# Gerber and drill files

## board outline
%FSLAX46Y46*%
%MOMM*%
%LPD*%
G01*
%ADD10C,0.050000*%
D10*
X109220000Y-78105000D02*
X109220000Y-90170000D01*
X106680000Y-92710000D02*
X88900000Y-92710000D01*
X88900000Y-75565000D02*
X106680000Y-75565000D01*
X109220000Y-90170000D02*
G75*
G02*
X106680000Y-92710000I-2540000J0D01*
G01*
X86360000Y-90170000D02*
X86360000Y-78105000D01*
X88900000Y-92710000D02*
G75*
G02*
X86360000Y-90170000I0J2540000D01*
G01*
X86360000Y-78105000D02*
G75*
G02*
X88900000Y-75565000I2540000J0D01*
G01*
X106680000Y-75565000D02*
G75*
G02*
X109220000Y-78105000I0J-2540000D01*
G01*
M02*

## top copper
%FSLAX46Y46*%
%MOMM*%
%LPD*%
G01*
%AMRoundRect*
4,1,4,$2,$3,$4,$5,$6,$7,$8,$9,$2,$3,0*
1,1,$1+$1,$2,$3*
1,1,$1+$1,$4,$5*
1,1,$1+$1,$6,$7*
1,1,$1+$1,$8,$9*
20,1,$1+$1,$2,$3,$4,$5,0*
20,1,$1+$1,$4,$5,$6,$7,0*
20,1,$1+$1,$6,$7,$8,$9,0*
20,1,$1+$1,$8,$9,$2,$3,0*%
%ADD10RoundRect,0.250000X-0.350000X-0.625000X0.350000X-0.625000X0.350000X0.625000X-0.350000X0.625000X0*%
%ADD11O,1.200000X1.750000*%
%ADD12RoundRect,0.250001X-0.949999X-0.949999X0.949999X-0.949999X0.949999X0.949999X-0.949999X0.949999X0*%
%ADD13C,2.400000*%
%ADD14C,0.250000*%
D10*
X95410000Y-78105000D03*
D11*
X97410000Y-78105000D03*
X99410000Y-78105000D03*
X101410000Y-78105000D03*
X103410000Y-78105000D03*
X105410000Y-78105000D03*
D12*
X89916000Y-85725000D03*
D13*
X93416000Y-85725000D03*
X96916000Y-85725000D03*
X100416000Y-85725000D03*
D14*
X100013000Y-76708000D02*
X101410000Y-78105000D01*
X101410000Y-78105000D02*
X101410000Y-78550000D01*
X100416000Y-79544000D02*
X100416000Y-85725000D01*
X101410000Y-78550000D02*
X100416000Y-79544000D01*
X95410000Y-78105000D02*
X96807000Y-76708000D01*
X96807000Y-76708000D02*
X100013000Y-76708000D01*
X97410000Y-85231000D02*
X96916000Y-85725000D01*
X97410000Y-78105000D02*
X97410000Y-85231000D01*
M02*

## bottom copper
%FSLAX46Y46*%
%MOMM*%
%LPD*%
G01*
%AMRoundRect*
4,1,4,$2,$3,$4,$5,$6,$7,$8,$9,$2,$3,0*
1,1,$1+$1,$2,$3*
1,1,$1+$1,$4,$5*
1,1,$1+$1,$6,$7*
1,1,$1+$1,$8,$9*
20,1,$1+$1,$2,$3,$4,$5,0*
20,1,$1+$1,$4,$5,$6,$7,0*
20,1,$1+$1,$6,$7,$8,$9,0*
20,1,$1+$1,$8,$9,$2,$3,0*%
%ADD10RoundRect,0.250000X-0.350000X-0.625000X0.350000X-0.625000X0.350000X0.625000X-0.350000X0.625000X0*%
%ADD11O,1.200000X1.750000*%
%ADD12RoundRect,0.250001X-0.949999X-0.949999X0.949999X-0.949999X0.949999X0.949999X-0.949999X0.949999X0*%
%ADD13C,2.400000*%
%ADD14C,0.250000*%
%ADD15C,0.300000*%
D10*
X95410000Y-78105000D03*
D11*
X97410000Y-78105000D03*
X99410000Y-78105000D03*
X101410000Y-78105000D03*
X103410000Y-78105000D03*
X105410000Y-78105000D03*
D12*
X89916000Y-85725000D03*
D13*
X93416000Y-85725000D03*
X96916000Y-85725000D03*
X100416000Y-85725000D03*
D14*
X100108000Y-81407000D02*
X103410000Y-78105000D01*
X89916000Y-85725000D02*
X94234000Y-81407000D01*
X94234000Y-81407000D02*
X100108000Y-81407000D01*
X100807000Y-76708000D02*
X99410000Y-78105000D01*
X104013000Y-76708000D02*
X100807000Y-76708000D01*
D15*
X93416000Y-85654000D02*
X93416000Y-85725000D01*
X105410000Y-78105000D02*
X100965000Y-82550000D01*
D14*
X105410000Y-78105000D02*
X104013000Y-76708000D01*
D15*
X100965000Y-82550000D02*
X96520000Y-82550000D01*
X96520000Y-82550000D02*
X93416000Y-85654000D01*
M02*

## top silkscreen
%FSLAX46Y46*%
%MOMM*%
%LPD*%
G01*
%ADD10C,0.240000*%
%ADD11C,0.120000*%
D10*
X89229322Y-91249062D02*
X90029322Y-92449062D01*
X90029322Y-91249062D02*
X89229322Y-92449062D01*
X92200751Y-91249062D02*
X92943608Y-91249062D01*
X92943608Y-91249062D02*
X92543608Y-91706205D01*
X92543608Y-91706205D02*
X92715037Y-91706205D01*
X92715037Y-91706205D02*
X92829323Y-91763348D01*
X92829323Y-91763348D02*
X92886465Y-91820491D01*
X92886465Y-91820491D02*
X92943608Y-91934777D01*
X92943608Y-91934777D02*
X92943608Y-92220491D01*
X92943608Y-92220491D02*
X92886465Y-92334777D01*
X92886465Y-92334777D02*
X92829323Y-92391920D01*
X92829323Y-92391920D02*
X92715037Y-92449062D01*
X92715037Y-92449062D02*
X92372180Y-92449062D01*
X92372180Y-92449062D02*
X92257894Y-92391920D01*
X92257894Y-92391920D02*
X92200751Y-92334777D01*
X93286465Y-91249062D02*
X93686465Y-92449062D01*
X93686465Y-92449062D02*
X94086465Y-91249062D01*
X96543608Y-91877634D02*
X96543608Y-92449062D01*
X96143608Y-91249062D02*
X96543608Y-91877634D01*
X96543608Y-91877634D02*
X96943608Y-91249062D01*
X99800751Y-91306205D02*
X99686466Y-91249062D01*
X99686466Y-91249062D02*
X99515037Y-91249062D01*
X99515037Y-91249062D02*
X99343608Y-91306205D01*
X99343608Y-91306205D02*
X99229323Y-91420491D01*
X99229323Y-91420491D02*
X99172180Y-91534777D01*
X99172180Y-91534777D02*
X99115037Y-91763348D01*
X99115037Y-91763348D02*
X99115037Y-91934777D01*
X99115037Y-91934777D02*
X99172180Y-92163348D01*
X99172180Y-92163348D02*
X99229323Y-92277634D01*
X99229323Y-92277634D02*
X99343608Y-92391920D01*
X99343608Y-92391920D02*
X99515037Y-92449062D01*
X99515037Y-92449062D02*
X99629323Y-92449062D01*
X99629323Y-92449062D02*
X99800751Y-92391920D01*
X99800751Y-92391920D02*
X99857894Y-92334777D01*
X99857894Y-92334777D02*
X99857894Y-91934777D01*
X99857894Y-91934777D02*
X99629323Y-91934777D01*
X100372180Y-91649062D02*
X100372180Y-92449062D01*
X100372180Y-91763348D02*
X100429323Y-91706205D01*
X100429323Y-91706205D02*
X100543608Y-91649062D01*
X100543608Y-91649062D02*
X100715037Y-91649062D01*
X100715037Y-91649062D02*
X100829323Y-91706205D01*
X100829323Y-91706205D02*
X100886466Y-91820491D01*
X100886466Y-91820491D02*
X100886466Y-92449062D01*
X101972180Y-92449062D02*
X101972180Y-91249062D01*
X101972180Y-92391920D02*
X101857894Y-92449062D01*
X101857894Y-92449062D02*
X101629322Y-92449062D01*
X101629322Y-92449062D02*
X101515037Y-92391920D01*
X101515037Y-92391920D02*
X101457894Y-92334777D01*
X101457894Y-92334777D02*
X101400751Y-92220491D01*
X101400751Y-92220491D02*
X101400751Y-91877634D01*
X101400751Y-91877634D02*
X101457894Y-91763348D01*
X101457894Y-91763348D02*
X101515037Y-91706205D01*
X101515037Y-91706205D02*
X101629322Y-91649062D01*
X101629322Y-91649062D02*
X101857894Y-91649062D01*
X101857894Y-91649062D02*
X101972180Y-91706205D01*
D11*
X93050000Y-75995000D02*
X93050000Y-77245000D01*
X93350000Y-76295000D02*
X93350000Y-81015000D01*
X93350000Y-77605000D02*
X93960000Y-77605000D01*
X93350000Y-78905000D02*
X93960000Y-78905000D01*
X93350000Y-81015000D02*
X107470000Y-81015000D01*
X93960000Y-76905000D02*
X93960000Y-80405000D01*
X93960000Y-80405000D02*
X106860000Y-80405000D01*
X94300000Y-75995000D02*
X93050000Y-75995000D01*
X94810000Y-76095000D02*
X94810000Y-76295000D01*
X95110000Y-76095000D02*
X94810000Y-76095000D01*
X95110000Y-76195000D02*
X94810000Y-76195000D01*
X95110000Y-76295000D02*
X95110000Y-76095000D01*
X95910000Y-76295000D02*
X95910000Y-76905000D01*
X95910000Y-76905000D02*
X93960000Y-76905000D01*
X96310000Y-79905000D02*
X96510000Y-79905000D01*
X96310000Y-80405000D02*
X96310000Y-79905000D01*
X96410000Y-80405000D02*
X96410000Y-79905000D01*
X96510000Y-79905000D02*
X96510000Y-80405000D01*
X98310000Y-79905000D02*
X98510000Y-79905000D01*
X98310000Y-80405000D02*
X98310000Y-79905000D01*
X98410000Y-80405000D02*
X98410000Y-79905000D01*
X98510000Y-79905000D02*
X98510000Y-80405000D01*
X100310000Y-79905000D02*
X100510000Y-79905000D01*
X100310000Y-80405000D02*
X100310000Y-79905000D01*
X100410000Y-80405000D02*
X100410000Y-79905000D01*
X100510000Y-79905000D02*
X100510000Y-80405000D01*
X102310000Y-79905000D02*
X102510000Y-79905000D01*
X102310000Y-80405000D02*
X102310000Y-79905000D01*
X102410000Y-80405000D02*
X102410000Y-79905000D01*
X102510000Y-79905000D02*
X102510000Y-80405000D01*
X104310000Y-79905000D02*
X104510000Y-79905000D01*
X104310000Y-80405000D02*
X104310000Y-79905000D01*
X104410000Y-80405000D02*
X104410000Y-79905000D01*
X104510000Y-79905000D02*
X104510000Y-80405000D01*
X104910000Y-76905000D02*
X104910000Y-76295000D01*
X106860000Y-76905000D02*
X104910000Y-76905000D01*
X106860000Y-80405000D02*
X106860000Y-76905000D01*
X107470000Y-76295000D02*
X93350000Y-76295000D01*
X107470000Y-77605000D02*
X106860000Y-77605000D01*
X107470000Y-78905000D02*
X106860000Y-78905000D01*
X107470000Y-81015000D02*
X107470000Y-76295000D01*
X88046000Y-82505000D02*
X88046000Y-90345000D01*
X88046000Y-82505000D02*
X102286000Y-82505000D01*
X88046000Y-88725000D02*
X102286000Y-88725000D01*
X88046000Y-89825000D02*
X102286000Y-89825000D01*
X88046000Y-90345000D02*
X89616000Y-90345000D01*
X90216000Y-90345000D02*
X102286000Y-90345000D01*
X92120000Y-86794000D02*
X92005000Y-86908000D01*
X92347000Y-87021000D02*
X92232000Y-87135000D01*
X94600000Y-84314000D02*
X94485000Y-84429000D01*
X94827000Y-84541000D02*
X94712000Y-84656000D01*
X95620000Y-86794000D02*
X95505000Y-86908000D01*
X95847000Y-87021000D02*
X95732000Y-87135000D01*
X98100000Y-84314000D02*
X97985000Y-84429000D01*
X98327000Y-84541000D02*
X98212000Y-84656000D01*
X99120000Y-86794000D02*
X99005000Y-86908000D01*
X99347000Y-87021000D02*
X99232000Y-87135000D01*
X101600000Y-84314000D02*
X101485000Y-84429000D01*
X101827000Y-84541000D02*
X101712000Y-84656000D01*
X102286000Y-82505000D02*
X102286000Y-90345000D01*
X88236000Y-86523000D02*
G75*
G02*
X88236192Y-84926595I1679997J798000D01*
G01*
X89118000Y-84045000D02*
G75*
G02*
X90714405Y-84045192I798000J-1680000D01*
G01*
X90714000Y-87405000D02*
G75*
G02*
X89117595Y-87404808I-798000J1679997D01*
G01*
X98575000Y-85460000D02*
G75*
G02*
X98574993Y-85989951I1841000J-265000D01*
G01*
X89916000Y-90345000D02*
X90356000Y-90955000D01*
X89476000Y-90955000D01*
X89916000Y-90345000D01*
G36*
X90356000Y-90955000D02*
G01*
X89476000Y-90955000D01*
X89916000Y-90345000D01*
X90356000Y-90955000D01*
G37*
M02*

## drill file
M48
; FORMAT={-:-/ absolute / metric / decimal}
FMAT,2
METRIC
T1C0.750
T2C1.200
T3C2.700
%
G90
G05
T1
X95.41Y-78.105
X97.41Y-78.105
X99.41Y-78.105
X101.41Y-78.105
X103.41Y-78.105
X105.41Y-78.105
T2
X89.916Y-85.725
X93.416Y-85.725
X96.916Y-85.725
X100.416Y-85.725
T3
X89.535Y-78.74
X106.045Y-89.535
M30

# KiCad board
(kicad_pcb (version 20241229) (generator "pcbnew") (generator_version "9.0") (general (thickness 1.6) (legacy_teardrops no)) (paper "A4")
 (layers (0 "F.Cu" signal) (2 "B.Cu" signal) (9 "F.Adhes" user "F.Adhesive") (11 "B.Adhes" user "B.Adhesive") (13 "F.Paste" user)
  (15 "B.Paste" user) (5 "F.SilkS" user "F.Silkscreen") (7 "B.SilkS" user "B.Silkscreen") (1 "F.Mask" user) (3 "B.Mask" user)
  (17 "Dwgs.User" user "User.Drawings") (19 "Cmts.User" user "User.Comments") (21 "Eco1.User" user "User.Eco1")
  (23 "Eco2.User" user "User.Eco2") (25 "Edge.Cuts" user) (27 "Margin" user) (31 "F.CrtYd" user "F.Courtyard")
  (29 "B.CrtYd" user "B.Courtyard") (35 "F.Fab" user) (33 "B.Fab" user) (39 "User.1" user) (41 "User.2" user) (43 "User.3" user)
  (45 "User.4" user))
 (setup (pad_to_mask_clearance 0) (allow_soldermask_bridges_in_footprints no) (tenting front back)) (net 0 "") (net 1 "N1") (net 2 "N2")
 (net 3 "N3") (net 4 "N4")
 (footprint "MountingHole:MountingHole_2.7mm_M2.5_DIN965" (layer "F.Cu") (at 89.535 78.74)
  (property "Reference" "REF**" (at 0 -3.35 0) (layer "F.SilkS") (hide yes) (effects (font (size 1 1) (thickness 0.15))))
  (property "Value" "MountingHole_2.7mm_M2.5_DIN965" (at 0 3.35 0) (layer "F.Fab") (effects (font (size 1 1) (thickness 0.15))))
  (pad "" np_thru_hole circle (at 0 0) (size 2.7 2.7) (drill 2.7) (layers "*.Cu" "*.Mask")))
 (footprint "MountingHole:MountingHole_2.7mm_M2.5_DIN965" (layer "F.Cu") (at 106.045 89.535)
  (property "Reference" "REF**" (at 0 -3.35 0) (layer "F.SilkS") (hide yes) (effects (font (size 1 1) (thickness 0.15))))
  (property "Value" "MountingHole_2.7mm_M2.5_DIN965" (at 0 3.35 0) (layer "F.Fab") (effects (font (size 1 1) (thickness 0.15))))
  (pad "" np_thru_hole circle (at 0 0) (size 2.7 2.7) (drill 2.7) (layers "*.Cu" "*.Mask")))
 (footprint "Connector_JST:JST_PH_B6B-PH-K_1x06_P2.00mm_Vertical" (layer "F.Cu") (at 95.41 78.105)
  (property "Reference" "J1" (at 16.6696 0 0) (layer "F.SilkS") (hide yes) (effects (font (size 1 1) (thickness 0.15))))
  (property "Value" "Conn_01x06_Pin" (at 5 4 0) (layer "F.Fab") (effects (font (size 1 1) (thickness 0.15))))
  (fp_line (start -2.36 -2.11) (end -2.36 -0.86) (stroke (width 0.12) (type solid)) (layer "F.SilkS"))
  (fp_line (start -2.06 -1.81) (end -2.06 2.91) (stroke (width 0.12) (type solid)) (layer "F.SilkS"))
  (fp_line (start -2.06 -0.5) (end -1.45 -0.5) (stroke (width 0.12) (type solid)) (layer "F.SilkS"))
  (fp_line (start -2.06 0.8) (end -1.45 0.8) (stroke (width 0.12) (type solid)) (layer "F.SilkS"))
  (fp_line (start -2.06 2.91) (end 12.06 2.91) (stroke (width 0.12) (type solid)) (layer "F.SilkS"))
  (fp_line (start -1.45 -1.2) (end -1.45 2.3) (stroke (width 0.12) (type solid)) (layer "F.SilkS"))
  (fp_line (start -1.45 2.3) (end 11.45 2.3) (stroke (width 0.12) (type solid)) (layer "F.SilkS"))
  (fp_line (start -1.11 -2.11) (end -2.36 -2.11) (stroke (width 0.12) (type solid)) (layer "F.SilkS"))
  (fp_line (start -0.6 -2.01) (end -0.6 -1.81) (stroke (width 0.12) (type solid)) (layer "F.SilkS"))
  (fp_line (start -0.3 -2.01) (end -0.6 -2.01) (stroke (width 0.12) (type solid)) (layer "F.SilkS"))
  (fp_line (start -0.3 -1.91) (end -0.6 -1.91) (stroke (width 0.12) (type solid)) (layer "F.SilkS"))
  (fp_line (start -0.3 -1.81) (end -0.3 -2.01) (stroke (width 0.12) (type solid)) (layer "F.SilkS"))
  (fp_line (start 0.5 -1.81) (end 0.5 -1.2) (stroke (width 0.12) (type solid)) (layer "F.SilkS"))
  (fp_line (start 0.5 -1.2) (end -1.45 -1.2) (stroke (width 0.12) (type solid)) (layer "F.SilkS"))
  (fp_line (start 0.9 1.8) (end 1.1 1.8) (stroke (width 0.12) (type solid)) (layer "F.SilkS"))
  (fp_line (start 0.9 2.3) (end 0.9 1.8) (stroke (width 0.12) (type solid)) (layer "F.SilkS"))
  (fp_line (start 1 2.3) (end 1 1.8) (stroke (width 0.12) (type solid)) (layer "F.SilkS"))
  (fp_line (start 1.1 1.8) (end 1.1 2.3) (stroke (width 0.12) (type solid)) (layer "F.SilkS"))
  (fp_line (start 2.9 1.8) (end 3.1 1.8) (stroke (width 0.12) (type solid)) (layer "F.SilkS"))
  (fp_line (start 2.9 2.3) (end 2.9 1.8) (stroke (width 0.12) (type solid)) (layer "F.SilkS"))
  (fp_line (start 3 2.3) (end 3 1.8) (stroke (width 0.12) (type solid)) (layer "F.SilkS"))
  (fp_line (start 3.1 1.8) (end 3.1 2.3) (stroke (width 0.12) (type solid)) (layer "F.SilkS"))
  (fp_line (start 4.9 1.8) (end 5.1 1.8) (stroke (width 0.12) (type solid)) (layer "F.SilkS"))
  (fp_line (start 4.9 2.3) (end 4.9 1.8) (stroke (width 0.12) (type solid)) (layer "F.SilkS"))
  (fp_line (start 5 2.3) (end 5 1.8) (stroke (width 0.12) (type solid)) (layer "F.SilkS"))
  (fp_line (start 5.1 1.8) (end 5.1 2.3) (stroke (width 0.12) (type solid)) (layer "F.SilkS"))
  (fp_line (start 6.9 1.8) (end 7.1 1.8) (stroke (width 0.12) (type solid)) (layer "F.SilkS"))
  (fp_line (start 6.9 2.3) (end 6.9 1.8) (stroke (width 0.12) (type solid)) (layer "F.SilkS"))
  (fp_line (start 7 2.3) (end 7 1.8) (stroke (width 0.12) (type solid)) (layer "F.SilkS"))
  (fp_line (start 7.1 1.8) (end 7.1 2.3) (stroke (width 0.12) (type solid)) (layer "F.SilkS"))
  (fp_line (start 8.9 1.8) (end 9.1 1.8) (stroke (width 0.12) (type solid)) (layer "F.SilkS"))
  (fp_line (start 8.9 2.3) (end 8.9 1.8) (stroke (width 0.12) (type solid)) (layer "F.SilkS"))
  (fp_line (start 9 2.3) (end 9 1.8) (stroke (width 0.12) (type solid)) (layer "F.SilkS"))
  (fp_line (start 9.1 1.8) (end 9.1 2.3) (stroke (width 0.12) (type solid)) (layer "F.SilkS"))
  (fp_line (start 9.5 -1.2) (end 9.5 -1.81) (stroke (width 0.12) (type solid)) (layer "F.SilkS"))
  (fp_line (start 11.45 -1.2) (end 9.5 -1.2) (stroke (width 0.12) (type solid)) (layer "F.SilkS"))
  (fp_line (start 11.45 2.3) (end 11.45 -1.2) (stroke (width 0.12) (type solid)) (layer "F.SilkS"))
  (fp_line (start 12.06 -1.81) (end -2.06 -1.81) (stroke (width 0.12) (type solid)) (layer "F.SilkS"))
  (fp_line (start 12.06 -0.5) (end 11.45 -0.5) (stroke (width 0.12) (type solid)) (layer "F.SilkS"))
  (fp_line (start 12.06 0.8) (end 11.45 0.8) (stroke (width 0.12) (type solid)) (layer "F.SilkS"))
  (fp_line (start 12.06 2.91) (end 12.06 -1.81) (stroke (width 0.12) (type solid)) (layer "F.SilkS"))
  (pad "1" thru_hole roundrect (at 0 0) (size 1.2 1.75) (drill 0.75) (layers "*.Cu" "*.Mask") (remove_unused_layers no)
   (roundrect_rratio 0.208333) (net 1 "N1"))
  (pad "2" thru_hole oval (at 2 0) (size 1.2 1.75) (drill 0.75) (layers "*.Cu" "*.Mask") (remove_unused_layers no) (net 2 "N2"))
  (pad "3" thru_hole oval (at 4 0) (size 1.2 1.75) (drill 0.75) (layers "*.Cu" "*.Mask") (remove_unused_layers no) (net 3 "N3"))
  (pad "4" thru_hole oval (at 6 0) (size 1.2 1.75) (drill 0.75) (layers "*.Cu" "*.Mask") (remove_unused_layers no) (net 1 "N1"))
  (pad "5" thru_hole oval (at 8 0) (size 1.2 1.75) (drill 0.75) (layers "*.Cu" "*.Mask") (remove_unused_layers no) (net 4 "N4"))
  (pad "6" thru_hole oval (at 10 0) (size 1.2 1.75) (drill 0.75) (layers "*.Cu" "*.Mask") (remove_unused_layers no) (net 3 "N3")))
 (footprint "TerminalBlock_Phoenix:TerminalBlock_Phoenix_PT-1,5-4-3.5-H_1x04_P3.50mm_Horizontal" (layer "F.Cu") (at 89.916 85.725)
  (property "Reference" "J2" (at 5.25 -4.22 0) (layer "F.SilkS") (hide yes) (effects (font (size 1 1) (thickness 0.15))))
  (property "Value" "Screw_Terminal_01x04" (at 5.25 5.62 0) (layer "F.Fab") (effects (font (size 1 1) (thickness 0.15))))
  (fp_line (start -1.87 -3.22) (end -1.87 4.62) (stroke (width 0.12) (type solid)) (layer "F.SilkS"))
  (fp_line (start -1.87 -3.22) (end 12.37 -3.22) (stroke (width 0.12) (type solid)) (layer "F.SilkS"))
  (fp_line (start -1.87 3) (end 12.37 3) (stroke (width 0.12) (type solid)) (layer "F.SilkS"))
  (fp_line (start -1.87 4.1) (end 12.37 4.1) (stroke (width 0.12) (type solid)) (layer "F.SilkS"))
  (fp_line (start -1.87 4.62) (end -0.3 4.62) (stroke (width 0.12) (type solid)) (layer "F.SilkS"))
  (fp_line (start 0.3 4.62) (end 12.37 4.62) (stroke (width 0.12) (type solid)) (layer "F.SilkS"))
  (fp_line (start 2.204 1.069) (end 2.089 1.183) (stroke (width 0.12) (type solid)) (layer "F.SilkS"))
  (fp_line (start 2.431 1.296) (end 2.316 1.41) (stroke (width 0.12) (type solid)) (layer "F.SilkS"))
  (fp_line (start 4.684 -1.411) (end 4.569 -1.296) (stroke (width 0.12) (type solid)) (layer "F.SilkS"))
  (fp_line (start 4.911 -1.184) (end 4.796 -1.069) (stroke (width 0.12) (type solid)) (layer "F.SilkS"))
  (fp_line (start 5.704 1.069) (end 5.589 1.183) (stroke (width 0.12) (type solid)) (layer "F.SilkS"))
  (fp_line (start 5.931 1.296) (end 5.816 1.41) (stroke (width 0.12) (type solid)) (layer "F.SilkS"))
  (fp_line (start 8.184 -1.411) (end 8.069 -1.296) (stroke (width 0.12) (type solid)) (layer "F.SilkS"))
  (fp_line (start 8.411 -1.184) (end 8.296 -1.069) (stroke (width 0.12) (type solid)) (layer "F.SilkS"))
  (fp_line (start 9.204 1.069) (end 9.089 1.183) (stroke (width 0.12) (type solid)) (layer "F.SilkS"))
  (fp_line (start 9.431 1.296) (end 9.316 1.41) (stroke (width 0.12) (type solid)) (layer "F.SilkS"))
  (fp_line (start 11.684 -1.411) (end 11.569 -1.296) (stroke (width 0.12) (type solid)) (layer "F.SilkS"))
  (fp_line (start 11.911 -1.184) (end 11.796 -1.069) (stroke (width 0.12) (type solid)) (layer "F.SilkS"))
  (fp_line (start 12.37 -3.22) (end 12.37 4.62) (stroke (width 0.12) (type solid)) (layer "F.SilkS"))
  (fp_arc (start -1.68 0.798) (mid -1.859894 -0.000224) (end -1.679808 -0.798405) (stroke (width 0.12) (type solid)) (layer "F.SilkS"))
  (fp_arc (start -0.798 -1.68) (mid 0.000224 -1.859894) (end 0.798405 -1.679808) (stroke (width 0.12) (type solid)) (layer "F.SilkS"))
  (fp_arc (start 0.798 1.68) (mid -0.000224 1.859894) (end -0.798405 1.679808) (stroke (width 0.12) (type solid)) (layer "F.SilkS"))
  (fp_arc (start 8.659 -0.265) (mid 12.359975 0.000025) (end 8.658993 0.264951) (stroke (width 0.12) (type solid)) (layer "F.SilkS"))
  (fp_poly (pts (xy 0 4.62) (xy 0.44 5.23) (xy -0.44 5.23) (xy 0 4.62)) (stroke (width 0.12) (type solid)) (fill yes) (layer "F.SilkS"))
  (pad "1" thru_hole roundrect (at 0 0) (size 2.4 2.4) (drill 1.2) (layers "*.Cu" "*.Mask") (remove_unused_layers no)
   (roundrect_rratio 0.104167) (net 4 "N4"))
  (pad "2" thru_hole circle (at 3.5 0) (size 2.4 2.4) (drill 1.2) (layers "*.Cu" "*.Mask") (remove_unused_layers no) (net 3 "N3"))
  (pad "3" thru_hole circle (at 7 0) (size 2.4 2.4) (drill 1.2) (layers "*.Cu" "*.Mask") (remove_unused_layers no) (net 2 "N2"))
  (pad "4" thru_hole circle (at 10.5 0) (size 2.4 2.4) (drill 1.2) (layers "*.Cu" "*.Mask") (remove_unused_layers no) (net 1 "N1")))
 (gr_line (start 109.22 78.105) (end 109.22 90.17) (stroke (width 0.05) (type default)) (layer "Edge.Cuts"))
 (gr_line (start 106.68 92.71) (end 88.9 92.71) (stroke (width 0.05) (type default)) (layer "Edge.Cuts"))
 (gr_line (start 88.9 75.565) (end 106.68 75.565) (stroke (width 0.05) (type default)) (layer "Edge.Cuts"))
 (gr_arc (start 109.22 90.17) (mid 108.476051 91.966051) (end 106.68 92.71) (stroke (width 0.05) (type default)) (layer "Edge.Cuts"))
 (gr_line (start 86.36 90.17) (end 86.36 78.105) (stroke (width 0.05) (type default)) (layer "Edge.Cuts"))
 (gr_arc (start 88.9 92.71) (mid 87.103949 91.966051) (end 86.36 90.17) (stroke (width 0.05) (type default)) (layer "Edge.Cuts"))
 (gr_arc (start 86.36 78.105) (mid 87.103949 76.308949) (end 88.9 75.565) (stroke (width 0.05) (type default)) (layer "Edge.Cuts"))
 (gr_arc (start 106.68 75.565) (mid 108.476051 76.308949) (end 109.22 78.105) (stroke (width 0.05) (type default)) (layer "Edge.Cuts"))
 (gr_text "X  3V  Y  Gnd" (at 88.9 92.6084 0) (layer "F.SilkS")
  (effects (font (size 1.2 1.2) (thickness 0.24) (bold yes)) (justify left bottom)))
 (segment (start 100.108 81.407) (end 103.41 78.105) (width 0.25) (layer "B.Cu") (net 4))
 (segment (start 89.916 85.725) (end 94.234 81.407) (width 0.25) (layer "B.Cu") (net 4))
 (segment (start 94.234 81.407) (end 100.108 81.407) (width 0.25) (layer "B.Cu") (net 4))
 (segment (start 100.807 76.708) (end 99.41 78.105) (width 0.25) (layer "B.Cu") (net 3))
 (segment (start 104.013 76.708) (end 100.807 76.708) (width 0.25) (layer "B.Cu") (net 3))
 (segment (start 93.416 85.654) (end 93.416 85.725) (width 0.3) (layer "B.Cu") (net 3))
 (segment (start 105.41 78.105) (end 100.965 82.55) (width 0.3) (layer "B.Cu") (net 3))
 (segment (start 105.41 78.105) (end 104.013 76.708) (width 0.25) (layer "B.Cu") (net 3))
 (segment (start 100.965 82.55) (end 96.52 82.55) (width 0.3) (layer "B.Cu") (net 3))
 (segment (start 96.52 82.55) (end 93.416 85.654) (width 0.3) (layer "B.Cu") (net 3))
 (segment (start 100.013 76.708) (end 101.41 78.105) (width 0.25) (layer "F.Cu") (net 1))
 (segment (start 101.41 78.105) (end 101.41 78.55) (width 0.25) (layer "F.Cu") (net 1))
 (segment (start 100.416 79.544) (end 100.416 85.725) (width 0.25) (layer "F.Cu") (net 1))
 (segment (start 101.41 78.55) (end 100.416 79.544) (width 0.25) (layer "F.Cu") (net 1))
 (segment (start 95.41 78.105) (end 96.807 76.708) (width 0.25) (layer "F.Cu") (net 1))
 (segment (start 96.807 76.708) (end 100.013 76.708) (width 0.25) (layer "F.Cu") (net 1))
 (segment (start 97.41 85.231) (end 96.916 85.725) (width 0.25) (layer "F.Cu") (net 2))
 (segment (start 97.41 78.105) (end 97.41 85.231) (width 0.25) (layer "F.Cu") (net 2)))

